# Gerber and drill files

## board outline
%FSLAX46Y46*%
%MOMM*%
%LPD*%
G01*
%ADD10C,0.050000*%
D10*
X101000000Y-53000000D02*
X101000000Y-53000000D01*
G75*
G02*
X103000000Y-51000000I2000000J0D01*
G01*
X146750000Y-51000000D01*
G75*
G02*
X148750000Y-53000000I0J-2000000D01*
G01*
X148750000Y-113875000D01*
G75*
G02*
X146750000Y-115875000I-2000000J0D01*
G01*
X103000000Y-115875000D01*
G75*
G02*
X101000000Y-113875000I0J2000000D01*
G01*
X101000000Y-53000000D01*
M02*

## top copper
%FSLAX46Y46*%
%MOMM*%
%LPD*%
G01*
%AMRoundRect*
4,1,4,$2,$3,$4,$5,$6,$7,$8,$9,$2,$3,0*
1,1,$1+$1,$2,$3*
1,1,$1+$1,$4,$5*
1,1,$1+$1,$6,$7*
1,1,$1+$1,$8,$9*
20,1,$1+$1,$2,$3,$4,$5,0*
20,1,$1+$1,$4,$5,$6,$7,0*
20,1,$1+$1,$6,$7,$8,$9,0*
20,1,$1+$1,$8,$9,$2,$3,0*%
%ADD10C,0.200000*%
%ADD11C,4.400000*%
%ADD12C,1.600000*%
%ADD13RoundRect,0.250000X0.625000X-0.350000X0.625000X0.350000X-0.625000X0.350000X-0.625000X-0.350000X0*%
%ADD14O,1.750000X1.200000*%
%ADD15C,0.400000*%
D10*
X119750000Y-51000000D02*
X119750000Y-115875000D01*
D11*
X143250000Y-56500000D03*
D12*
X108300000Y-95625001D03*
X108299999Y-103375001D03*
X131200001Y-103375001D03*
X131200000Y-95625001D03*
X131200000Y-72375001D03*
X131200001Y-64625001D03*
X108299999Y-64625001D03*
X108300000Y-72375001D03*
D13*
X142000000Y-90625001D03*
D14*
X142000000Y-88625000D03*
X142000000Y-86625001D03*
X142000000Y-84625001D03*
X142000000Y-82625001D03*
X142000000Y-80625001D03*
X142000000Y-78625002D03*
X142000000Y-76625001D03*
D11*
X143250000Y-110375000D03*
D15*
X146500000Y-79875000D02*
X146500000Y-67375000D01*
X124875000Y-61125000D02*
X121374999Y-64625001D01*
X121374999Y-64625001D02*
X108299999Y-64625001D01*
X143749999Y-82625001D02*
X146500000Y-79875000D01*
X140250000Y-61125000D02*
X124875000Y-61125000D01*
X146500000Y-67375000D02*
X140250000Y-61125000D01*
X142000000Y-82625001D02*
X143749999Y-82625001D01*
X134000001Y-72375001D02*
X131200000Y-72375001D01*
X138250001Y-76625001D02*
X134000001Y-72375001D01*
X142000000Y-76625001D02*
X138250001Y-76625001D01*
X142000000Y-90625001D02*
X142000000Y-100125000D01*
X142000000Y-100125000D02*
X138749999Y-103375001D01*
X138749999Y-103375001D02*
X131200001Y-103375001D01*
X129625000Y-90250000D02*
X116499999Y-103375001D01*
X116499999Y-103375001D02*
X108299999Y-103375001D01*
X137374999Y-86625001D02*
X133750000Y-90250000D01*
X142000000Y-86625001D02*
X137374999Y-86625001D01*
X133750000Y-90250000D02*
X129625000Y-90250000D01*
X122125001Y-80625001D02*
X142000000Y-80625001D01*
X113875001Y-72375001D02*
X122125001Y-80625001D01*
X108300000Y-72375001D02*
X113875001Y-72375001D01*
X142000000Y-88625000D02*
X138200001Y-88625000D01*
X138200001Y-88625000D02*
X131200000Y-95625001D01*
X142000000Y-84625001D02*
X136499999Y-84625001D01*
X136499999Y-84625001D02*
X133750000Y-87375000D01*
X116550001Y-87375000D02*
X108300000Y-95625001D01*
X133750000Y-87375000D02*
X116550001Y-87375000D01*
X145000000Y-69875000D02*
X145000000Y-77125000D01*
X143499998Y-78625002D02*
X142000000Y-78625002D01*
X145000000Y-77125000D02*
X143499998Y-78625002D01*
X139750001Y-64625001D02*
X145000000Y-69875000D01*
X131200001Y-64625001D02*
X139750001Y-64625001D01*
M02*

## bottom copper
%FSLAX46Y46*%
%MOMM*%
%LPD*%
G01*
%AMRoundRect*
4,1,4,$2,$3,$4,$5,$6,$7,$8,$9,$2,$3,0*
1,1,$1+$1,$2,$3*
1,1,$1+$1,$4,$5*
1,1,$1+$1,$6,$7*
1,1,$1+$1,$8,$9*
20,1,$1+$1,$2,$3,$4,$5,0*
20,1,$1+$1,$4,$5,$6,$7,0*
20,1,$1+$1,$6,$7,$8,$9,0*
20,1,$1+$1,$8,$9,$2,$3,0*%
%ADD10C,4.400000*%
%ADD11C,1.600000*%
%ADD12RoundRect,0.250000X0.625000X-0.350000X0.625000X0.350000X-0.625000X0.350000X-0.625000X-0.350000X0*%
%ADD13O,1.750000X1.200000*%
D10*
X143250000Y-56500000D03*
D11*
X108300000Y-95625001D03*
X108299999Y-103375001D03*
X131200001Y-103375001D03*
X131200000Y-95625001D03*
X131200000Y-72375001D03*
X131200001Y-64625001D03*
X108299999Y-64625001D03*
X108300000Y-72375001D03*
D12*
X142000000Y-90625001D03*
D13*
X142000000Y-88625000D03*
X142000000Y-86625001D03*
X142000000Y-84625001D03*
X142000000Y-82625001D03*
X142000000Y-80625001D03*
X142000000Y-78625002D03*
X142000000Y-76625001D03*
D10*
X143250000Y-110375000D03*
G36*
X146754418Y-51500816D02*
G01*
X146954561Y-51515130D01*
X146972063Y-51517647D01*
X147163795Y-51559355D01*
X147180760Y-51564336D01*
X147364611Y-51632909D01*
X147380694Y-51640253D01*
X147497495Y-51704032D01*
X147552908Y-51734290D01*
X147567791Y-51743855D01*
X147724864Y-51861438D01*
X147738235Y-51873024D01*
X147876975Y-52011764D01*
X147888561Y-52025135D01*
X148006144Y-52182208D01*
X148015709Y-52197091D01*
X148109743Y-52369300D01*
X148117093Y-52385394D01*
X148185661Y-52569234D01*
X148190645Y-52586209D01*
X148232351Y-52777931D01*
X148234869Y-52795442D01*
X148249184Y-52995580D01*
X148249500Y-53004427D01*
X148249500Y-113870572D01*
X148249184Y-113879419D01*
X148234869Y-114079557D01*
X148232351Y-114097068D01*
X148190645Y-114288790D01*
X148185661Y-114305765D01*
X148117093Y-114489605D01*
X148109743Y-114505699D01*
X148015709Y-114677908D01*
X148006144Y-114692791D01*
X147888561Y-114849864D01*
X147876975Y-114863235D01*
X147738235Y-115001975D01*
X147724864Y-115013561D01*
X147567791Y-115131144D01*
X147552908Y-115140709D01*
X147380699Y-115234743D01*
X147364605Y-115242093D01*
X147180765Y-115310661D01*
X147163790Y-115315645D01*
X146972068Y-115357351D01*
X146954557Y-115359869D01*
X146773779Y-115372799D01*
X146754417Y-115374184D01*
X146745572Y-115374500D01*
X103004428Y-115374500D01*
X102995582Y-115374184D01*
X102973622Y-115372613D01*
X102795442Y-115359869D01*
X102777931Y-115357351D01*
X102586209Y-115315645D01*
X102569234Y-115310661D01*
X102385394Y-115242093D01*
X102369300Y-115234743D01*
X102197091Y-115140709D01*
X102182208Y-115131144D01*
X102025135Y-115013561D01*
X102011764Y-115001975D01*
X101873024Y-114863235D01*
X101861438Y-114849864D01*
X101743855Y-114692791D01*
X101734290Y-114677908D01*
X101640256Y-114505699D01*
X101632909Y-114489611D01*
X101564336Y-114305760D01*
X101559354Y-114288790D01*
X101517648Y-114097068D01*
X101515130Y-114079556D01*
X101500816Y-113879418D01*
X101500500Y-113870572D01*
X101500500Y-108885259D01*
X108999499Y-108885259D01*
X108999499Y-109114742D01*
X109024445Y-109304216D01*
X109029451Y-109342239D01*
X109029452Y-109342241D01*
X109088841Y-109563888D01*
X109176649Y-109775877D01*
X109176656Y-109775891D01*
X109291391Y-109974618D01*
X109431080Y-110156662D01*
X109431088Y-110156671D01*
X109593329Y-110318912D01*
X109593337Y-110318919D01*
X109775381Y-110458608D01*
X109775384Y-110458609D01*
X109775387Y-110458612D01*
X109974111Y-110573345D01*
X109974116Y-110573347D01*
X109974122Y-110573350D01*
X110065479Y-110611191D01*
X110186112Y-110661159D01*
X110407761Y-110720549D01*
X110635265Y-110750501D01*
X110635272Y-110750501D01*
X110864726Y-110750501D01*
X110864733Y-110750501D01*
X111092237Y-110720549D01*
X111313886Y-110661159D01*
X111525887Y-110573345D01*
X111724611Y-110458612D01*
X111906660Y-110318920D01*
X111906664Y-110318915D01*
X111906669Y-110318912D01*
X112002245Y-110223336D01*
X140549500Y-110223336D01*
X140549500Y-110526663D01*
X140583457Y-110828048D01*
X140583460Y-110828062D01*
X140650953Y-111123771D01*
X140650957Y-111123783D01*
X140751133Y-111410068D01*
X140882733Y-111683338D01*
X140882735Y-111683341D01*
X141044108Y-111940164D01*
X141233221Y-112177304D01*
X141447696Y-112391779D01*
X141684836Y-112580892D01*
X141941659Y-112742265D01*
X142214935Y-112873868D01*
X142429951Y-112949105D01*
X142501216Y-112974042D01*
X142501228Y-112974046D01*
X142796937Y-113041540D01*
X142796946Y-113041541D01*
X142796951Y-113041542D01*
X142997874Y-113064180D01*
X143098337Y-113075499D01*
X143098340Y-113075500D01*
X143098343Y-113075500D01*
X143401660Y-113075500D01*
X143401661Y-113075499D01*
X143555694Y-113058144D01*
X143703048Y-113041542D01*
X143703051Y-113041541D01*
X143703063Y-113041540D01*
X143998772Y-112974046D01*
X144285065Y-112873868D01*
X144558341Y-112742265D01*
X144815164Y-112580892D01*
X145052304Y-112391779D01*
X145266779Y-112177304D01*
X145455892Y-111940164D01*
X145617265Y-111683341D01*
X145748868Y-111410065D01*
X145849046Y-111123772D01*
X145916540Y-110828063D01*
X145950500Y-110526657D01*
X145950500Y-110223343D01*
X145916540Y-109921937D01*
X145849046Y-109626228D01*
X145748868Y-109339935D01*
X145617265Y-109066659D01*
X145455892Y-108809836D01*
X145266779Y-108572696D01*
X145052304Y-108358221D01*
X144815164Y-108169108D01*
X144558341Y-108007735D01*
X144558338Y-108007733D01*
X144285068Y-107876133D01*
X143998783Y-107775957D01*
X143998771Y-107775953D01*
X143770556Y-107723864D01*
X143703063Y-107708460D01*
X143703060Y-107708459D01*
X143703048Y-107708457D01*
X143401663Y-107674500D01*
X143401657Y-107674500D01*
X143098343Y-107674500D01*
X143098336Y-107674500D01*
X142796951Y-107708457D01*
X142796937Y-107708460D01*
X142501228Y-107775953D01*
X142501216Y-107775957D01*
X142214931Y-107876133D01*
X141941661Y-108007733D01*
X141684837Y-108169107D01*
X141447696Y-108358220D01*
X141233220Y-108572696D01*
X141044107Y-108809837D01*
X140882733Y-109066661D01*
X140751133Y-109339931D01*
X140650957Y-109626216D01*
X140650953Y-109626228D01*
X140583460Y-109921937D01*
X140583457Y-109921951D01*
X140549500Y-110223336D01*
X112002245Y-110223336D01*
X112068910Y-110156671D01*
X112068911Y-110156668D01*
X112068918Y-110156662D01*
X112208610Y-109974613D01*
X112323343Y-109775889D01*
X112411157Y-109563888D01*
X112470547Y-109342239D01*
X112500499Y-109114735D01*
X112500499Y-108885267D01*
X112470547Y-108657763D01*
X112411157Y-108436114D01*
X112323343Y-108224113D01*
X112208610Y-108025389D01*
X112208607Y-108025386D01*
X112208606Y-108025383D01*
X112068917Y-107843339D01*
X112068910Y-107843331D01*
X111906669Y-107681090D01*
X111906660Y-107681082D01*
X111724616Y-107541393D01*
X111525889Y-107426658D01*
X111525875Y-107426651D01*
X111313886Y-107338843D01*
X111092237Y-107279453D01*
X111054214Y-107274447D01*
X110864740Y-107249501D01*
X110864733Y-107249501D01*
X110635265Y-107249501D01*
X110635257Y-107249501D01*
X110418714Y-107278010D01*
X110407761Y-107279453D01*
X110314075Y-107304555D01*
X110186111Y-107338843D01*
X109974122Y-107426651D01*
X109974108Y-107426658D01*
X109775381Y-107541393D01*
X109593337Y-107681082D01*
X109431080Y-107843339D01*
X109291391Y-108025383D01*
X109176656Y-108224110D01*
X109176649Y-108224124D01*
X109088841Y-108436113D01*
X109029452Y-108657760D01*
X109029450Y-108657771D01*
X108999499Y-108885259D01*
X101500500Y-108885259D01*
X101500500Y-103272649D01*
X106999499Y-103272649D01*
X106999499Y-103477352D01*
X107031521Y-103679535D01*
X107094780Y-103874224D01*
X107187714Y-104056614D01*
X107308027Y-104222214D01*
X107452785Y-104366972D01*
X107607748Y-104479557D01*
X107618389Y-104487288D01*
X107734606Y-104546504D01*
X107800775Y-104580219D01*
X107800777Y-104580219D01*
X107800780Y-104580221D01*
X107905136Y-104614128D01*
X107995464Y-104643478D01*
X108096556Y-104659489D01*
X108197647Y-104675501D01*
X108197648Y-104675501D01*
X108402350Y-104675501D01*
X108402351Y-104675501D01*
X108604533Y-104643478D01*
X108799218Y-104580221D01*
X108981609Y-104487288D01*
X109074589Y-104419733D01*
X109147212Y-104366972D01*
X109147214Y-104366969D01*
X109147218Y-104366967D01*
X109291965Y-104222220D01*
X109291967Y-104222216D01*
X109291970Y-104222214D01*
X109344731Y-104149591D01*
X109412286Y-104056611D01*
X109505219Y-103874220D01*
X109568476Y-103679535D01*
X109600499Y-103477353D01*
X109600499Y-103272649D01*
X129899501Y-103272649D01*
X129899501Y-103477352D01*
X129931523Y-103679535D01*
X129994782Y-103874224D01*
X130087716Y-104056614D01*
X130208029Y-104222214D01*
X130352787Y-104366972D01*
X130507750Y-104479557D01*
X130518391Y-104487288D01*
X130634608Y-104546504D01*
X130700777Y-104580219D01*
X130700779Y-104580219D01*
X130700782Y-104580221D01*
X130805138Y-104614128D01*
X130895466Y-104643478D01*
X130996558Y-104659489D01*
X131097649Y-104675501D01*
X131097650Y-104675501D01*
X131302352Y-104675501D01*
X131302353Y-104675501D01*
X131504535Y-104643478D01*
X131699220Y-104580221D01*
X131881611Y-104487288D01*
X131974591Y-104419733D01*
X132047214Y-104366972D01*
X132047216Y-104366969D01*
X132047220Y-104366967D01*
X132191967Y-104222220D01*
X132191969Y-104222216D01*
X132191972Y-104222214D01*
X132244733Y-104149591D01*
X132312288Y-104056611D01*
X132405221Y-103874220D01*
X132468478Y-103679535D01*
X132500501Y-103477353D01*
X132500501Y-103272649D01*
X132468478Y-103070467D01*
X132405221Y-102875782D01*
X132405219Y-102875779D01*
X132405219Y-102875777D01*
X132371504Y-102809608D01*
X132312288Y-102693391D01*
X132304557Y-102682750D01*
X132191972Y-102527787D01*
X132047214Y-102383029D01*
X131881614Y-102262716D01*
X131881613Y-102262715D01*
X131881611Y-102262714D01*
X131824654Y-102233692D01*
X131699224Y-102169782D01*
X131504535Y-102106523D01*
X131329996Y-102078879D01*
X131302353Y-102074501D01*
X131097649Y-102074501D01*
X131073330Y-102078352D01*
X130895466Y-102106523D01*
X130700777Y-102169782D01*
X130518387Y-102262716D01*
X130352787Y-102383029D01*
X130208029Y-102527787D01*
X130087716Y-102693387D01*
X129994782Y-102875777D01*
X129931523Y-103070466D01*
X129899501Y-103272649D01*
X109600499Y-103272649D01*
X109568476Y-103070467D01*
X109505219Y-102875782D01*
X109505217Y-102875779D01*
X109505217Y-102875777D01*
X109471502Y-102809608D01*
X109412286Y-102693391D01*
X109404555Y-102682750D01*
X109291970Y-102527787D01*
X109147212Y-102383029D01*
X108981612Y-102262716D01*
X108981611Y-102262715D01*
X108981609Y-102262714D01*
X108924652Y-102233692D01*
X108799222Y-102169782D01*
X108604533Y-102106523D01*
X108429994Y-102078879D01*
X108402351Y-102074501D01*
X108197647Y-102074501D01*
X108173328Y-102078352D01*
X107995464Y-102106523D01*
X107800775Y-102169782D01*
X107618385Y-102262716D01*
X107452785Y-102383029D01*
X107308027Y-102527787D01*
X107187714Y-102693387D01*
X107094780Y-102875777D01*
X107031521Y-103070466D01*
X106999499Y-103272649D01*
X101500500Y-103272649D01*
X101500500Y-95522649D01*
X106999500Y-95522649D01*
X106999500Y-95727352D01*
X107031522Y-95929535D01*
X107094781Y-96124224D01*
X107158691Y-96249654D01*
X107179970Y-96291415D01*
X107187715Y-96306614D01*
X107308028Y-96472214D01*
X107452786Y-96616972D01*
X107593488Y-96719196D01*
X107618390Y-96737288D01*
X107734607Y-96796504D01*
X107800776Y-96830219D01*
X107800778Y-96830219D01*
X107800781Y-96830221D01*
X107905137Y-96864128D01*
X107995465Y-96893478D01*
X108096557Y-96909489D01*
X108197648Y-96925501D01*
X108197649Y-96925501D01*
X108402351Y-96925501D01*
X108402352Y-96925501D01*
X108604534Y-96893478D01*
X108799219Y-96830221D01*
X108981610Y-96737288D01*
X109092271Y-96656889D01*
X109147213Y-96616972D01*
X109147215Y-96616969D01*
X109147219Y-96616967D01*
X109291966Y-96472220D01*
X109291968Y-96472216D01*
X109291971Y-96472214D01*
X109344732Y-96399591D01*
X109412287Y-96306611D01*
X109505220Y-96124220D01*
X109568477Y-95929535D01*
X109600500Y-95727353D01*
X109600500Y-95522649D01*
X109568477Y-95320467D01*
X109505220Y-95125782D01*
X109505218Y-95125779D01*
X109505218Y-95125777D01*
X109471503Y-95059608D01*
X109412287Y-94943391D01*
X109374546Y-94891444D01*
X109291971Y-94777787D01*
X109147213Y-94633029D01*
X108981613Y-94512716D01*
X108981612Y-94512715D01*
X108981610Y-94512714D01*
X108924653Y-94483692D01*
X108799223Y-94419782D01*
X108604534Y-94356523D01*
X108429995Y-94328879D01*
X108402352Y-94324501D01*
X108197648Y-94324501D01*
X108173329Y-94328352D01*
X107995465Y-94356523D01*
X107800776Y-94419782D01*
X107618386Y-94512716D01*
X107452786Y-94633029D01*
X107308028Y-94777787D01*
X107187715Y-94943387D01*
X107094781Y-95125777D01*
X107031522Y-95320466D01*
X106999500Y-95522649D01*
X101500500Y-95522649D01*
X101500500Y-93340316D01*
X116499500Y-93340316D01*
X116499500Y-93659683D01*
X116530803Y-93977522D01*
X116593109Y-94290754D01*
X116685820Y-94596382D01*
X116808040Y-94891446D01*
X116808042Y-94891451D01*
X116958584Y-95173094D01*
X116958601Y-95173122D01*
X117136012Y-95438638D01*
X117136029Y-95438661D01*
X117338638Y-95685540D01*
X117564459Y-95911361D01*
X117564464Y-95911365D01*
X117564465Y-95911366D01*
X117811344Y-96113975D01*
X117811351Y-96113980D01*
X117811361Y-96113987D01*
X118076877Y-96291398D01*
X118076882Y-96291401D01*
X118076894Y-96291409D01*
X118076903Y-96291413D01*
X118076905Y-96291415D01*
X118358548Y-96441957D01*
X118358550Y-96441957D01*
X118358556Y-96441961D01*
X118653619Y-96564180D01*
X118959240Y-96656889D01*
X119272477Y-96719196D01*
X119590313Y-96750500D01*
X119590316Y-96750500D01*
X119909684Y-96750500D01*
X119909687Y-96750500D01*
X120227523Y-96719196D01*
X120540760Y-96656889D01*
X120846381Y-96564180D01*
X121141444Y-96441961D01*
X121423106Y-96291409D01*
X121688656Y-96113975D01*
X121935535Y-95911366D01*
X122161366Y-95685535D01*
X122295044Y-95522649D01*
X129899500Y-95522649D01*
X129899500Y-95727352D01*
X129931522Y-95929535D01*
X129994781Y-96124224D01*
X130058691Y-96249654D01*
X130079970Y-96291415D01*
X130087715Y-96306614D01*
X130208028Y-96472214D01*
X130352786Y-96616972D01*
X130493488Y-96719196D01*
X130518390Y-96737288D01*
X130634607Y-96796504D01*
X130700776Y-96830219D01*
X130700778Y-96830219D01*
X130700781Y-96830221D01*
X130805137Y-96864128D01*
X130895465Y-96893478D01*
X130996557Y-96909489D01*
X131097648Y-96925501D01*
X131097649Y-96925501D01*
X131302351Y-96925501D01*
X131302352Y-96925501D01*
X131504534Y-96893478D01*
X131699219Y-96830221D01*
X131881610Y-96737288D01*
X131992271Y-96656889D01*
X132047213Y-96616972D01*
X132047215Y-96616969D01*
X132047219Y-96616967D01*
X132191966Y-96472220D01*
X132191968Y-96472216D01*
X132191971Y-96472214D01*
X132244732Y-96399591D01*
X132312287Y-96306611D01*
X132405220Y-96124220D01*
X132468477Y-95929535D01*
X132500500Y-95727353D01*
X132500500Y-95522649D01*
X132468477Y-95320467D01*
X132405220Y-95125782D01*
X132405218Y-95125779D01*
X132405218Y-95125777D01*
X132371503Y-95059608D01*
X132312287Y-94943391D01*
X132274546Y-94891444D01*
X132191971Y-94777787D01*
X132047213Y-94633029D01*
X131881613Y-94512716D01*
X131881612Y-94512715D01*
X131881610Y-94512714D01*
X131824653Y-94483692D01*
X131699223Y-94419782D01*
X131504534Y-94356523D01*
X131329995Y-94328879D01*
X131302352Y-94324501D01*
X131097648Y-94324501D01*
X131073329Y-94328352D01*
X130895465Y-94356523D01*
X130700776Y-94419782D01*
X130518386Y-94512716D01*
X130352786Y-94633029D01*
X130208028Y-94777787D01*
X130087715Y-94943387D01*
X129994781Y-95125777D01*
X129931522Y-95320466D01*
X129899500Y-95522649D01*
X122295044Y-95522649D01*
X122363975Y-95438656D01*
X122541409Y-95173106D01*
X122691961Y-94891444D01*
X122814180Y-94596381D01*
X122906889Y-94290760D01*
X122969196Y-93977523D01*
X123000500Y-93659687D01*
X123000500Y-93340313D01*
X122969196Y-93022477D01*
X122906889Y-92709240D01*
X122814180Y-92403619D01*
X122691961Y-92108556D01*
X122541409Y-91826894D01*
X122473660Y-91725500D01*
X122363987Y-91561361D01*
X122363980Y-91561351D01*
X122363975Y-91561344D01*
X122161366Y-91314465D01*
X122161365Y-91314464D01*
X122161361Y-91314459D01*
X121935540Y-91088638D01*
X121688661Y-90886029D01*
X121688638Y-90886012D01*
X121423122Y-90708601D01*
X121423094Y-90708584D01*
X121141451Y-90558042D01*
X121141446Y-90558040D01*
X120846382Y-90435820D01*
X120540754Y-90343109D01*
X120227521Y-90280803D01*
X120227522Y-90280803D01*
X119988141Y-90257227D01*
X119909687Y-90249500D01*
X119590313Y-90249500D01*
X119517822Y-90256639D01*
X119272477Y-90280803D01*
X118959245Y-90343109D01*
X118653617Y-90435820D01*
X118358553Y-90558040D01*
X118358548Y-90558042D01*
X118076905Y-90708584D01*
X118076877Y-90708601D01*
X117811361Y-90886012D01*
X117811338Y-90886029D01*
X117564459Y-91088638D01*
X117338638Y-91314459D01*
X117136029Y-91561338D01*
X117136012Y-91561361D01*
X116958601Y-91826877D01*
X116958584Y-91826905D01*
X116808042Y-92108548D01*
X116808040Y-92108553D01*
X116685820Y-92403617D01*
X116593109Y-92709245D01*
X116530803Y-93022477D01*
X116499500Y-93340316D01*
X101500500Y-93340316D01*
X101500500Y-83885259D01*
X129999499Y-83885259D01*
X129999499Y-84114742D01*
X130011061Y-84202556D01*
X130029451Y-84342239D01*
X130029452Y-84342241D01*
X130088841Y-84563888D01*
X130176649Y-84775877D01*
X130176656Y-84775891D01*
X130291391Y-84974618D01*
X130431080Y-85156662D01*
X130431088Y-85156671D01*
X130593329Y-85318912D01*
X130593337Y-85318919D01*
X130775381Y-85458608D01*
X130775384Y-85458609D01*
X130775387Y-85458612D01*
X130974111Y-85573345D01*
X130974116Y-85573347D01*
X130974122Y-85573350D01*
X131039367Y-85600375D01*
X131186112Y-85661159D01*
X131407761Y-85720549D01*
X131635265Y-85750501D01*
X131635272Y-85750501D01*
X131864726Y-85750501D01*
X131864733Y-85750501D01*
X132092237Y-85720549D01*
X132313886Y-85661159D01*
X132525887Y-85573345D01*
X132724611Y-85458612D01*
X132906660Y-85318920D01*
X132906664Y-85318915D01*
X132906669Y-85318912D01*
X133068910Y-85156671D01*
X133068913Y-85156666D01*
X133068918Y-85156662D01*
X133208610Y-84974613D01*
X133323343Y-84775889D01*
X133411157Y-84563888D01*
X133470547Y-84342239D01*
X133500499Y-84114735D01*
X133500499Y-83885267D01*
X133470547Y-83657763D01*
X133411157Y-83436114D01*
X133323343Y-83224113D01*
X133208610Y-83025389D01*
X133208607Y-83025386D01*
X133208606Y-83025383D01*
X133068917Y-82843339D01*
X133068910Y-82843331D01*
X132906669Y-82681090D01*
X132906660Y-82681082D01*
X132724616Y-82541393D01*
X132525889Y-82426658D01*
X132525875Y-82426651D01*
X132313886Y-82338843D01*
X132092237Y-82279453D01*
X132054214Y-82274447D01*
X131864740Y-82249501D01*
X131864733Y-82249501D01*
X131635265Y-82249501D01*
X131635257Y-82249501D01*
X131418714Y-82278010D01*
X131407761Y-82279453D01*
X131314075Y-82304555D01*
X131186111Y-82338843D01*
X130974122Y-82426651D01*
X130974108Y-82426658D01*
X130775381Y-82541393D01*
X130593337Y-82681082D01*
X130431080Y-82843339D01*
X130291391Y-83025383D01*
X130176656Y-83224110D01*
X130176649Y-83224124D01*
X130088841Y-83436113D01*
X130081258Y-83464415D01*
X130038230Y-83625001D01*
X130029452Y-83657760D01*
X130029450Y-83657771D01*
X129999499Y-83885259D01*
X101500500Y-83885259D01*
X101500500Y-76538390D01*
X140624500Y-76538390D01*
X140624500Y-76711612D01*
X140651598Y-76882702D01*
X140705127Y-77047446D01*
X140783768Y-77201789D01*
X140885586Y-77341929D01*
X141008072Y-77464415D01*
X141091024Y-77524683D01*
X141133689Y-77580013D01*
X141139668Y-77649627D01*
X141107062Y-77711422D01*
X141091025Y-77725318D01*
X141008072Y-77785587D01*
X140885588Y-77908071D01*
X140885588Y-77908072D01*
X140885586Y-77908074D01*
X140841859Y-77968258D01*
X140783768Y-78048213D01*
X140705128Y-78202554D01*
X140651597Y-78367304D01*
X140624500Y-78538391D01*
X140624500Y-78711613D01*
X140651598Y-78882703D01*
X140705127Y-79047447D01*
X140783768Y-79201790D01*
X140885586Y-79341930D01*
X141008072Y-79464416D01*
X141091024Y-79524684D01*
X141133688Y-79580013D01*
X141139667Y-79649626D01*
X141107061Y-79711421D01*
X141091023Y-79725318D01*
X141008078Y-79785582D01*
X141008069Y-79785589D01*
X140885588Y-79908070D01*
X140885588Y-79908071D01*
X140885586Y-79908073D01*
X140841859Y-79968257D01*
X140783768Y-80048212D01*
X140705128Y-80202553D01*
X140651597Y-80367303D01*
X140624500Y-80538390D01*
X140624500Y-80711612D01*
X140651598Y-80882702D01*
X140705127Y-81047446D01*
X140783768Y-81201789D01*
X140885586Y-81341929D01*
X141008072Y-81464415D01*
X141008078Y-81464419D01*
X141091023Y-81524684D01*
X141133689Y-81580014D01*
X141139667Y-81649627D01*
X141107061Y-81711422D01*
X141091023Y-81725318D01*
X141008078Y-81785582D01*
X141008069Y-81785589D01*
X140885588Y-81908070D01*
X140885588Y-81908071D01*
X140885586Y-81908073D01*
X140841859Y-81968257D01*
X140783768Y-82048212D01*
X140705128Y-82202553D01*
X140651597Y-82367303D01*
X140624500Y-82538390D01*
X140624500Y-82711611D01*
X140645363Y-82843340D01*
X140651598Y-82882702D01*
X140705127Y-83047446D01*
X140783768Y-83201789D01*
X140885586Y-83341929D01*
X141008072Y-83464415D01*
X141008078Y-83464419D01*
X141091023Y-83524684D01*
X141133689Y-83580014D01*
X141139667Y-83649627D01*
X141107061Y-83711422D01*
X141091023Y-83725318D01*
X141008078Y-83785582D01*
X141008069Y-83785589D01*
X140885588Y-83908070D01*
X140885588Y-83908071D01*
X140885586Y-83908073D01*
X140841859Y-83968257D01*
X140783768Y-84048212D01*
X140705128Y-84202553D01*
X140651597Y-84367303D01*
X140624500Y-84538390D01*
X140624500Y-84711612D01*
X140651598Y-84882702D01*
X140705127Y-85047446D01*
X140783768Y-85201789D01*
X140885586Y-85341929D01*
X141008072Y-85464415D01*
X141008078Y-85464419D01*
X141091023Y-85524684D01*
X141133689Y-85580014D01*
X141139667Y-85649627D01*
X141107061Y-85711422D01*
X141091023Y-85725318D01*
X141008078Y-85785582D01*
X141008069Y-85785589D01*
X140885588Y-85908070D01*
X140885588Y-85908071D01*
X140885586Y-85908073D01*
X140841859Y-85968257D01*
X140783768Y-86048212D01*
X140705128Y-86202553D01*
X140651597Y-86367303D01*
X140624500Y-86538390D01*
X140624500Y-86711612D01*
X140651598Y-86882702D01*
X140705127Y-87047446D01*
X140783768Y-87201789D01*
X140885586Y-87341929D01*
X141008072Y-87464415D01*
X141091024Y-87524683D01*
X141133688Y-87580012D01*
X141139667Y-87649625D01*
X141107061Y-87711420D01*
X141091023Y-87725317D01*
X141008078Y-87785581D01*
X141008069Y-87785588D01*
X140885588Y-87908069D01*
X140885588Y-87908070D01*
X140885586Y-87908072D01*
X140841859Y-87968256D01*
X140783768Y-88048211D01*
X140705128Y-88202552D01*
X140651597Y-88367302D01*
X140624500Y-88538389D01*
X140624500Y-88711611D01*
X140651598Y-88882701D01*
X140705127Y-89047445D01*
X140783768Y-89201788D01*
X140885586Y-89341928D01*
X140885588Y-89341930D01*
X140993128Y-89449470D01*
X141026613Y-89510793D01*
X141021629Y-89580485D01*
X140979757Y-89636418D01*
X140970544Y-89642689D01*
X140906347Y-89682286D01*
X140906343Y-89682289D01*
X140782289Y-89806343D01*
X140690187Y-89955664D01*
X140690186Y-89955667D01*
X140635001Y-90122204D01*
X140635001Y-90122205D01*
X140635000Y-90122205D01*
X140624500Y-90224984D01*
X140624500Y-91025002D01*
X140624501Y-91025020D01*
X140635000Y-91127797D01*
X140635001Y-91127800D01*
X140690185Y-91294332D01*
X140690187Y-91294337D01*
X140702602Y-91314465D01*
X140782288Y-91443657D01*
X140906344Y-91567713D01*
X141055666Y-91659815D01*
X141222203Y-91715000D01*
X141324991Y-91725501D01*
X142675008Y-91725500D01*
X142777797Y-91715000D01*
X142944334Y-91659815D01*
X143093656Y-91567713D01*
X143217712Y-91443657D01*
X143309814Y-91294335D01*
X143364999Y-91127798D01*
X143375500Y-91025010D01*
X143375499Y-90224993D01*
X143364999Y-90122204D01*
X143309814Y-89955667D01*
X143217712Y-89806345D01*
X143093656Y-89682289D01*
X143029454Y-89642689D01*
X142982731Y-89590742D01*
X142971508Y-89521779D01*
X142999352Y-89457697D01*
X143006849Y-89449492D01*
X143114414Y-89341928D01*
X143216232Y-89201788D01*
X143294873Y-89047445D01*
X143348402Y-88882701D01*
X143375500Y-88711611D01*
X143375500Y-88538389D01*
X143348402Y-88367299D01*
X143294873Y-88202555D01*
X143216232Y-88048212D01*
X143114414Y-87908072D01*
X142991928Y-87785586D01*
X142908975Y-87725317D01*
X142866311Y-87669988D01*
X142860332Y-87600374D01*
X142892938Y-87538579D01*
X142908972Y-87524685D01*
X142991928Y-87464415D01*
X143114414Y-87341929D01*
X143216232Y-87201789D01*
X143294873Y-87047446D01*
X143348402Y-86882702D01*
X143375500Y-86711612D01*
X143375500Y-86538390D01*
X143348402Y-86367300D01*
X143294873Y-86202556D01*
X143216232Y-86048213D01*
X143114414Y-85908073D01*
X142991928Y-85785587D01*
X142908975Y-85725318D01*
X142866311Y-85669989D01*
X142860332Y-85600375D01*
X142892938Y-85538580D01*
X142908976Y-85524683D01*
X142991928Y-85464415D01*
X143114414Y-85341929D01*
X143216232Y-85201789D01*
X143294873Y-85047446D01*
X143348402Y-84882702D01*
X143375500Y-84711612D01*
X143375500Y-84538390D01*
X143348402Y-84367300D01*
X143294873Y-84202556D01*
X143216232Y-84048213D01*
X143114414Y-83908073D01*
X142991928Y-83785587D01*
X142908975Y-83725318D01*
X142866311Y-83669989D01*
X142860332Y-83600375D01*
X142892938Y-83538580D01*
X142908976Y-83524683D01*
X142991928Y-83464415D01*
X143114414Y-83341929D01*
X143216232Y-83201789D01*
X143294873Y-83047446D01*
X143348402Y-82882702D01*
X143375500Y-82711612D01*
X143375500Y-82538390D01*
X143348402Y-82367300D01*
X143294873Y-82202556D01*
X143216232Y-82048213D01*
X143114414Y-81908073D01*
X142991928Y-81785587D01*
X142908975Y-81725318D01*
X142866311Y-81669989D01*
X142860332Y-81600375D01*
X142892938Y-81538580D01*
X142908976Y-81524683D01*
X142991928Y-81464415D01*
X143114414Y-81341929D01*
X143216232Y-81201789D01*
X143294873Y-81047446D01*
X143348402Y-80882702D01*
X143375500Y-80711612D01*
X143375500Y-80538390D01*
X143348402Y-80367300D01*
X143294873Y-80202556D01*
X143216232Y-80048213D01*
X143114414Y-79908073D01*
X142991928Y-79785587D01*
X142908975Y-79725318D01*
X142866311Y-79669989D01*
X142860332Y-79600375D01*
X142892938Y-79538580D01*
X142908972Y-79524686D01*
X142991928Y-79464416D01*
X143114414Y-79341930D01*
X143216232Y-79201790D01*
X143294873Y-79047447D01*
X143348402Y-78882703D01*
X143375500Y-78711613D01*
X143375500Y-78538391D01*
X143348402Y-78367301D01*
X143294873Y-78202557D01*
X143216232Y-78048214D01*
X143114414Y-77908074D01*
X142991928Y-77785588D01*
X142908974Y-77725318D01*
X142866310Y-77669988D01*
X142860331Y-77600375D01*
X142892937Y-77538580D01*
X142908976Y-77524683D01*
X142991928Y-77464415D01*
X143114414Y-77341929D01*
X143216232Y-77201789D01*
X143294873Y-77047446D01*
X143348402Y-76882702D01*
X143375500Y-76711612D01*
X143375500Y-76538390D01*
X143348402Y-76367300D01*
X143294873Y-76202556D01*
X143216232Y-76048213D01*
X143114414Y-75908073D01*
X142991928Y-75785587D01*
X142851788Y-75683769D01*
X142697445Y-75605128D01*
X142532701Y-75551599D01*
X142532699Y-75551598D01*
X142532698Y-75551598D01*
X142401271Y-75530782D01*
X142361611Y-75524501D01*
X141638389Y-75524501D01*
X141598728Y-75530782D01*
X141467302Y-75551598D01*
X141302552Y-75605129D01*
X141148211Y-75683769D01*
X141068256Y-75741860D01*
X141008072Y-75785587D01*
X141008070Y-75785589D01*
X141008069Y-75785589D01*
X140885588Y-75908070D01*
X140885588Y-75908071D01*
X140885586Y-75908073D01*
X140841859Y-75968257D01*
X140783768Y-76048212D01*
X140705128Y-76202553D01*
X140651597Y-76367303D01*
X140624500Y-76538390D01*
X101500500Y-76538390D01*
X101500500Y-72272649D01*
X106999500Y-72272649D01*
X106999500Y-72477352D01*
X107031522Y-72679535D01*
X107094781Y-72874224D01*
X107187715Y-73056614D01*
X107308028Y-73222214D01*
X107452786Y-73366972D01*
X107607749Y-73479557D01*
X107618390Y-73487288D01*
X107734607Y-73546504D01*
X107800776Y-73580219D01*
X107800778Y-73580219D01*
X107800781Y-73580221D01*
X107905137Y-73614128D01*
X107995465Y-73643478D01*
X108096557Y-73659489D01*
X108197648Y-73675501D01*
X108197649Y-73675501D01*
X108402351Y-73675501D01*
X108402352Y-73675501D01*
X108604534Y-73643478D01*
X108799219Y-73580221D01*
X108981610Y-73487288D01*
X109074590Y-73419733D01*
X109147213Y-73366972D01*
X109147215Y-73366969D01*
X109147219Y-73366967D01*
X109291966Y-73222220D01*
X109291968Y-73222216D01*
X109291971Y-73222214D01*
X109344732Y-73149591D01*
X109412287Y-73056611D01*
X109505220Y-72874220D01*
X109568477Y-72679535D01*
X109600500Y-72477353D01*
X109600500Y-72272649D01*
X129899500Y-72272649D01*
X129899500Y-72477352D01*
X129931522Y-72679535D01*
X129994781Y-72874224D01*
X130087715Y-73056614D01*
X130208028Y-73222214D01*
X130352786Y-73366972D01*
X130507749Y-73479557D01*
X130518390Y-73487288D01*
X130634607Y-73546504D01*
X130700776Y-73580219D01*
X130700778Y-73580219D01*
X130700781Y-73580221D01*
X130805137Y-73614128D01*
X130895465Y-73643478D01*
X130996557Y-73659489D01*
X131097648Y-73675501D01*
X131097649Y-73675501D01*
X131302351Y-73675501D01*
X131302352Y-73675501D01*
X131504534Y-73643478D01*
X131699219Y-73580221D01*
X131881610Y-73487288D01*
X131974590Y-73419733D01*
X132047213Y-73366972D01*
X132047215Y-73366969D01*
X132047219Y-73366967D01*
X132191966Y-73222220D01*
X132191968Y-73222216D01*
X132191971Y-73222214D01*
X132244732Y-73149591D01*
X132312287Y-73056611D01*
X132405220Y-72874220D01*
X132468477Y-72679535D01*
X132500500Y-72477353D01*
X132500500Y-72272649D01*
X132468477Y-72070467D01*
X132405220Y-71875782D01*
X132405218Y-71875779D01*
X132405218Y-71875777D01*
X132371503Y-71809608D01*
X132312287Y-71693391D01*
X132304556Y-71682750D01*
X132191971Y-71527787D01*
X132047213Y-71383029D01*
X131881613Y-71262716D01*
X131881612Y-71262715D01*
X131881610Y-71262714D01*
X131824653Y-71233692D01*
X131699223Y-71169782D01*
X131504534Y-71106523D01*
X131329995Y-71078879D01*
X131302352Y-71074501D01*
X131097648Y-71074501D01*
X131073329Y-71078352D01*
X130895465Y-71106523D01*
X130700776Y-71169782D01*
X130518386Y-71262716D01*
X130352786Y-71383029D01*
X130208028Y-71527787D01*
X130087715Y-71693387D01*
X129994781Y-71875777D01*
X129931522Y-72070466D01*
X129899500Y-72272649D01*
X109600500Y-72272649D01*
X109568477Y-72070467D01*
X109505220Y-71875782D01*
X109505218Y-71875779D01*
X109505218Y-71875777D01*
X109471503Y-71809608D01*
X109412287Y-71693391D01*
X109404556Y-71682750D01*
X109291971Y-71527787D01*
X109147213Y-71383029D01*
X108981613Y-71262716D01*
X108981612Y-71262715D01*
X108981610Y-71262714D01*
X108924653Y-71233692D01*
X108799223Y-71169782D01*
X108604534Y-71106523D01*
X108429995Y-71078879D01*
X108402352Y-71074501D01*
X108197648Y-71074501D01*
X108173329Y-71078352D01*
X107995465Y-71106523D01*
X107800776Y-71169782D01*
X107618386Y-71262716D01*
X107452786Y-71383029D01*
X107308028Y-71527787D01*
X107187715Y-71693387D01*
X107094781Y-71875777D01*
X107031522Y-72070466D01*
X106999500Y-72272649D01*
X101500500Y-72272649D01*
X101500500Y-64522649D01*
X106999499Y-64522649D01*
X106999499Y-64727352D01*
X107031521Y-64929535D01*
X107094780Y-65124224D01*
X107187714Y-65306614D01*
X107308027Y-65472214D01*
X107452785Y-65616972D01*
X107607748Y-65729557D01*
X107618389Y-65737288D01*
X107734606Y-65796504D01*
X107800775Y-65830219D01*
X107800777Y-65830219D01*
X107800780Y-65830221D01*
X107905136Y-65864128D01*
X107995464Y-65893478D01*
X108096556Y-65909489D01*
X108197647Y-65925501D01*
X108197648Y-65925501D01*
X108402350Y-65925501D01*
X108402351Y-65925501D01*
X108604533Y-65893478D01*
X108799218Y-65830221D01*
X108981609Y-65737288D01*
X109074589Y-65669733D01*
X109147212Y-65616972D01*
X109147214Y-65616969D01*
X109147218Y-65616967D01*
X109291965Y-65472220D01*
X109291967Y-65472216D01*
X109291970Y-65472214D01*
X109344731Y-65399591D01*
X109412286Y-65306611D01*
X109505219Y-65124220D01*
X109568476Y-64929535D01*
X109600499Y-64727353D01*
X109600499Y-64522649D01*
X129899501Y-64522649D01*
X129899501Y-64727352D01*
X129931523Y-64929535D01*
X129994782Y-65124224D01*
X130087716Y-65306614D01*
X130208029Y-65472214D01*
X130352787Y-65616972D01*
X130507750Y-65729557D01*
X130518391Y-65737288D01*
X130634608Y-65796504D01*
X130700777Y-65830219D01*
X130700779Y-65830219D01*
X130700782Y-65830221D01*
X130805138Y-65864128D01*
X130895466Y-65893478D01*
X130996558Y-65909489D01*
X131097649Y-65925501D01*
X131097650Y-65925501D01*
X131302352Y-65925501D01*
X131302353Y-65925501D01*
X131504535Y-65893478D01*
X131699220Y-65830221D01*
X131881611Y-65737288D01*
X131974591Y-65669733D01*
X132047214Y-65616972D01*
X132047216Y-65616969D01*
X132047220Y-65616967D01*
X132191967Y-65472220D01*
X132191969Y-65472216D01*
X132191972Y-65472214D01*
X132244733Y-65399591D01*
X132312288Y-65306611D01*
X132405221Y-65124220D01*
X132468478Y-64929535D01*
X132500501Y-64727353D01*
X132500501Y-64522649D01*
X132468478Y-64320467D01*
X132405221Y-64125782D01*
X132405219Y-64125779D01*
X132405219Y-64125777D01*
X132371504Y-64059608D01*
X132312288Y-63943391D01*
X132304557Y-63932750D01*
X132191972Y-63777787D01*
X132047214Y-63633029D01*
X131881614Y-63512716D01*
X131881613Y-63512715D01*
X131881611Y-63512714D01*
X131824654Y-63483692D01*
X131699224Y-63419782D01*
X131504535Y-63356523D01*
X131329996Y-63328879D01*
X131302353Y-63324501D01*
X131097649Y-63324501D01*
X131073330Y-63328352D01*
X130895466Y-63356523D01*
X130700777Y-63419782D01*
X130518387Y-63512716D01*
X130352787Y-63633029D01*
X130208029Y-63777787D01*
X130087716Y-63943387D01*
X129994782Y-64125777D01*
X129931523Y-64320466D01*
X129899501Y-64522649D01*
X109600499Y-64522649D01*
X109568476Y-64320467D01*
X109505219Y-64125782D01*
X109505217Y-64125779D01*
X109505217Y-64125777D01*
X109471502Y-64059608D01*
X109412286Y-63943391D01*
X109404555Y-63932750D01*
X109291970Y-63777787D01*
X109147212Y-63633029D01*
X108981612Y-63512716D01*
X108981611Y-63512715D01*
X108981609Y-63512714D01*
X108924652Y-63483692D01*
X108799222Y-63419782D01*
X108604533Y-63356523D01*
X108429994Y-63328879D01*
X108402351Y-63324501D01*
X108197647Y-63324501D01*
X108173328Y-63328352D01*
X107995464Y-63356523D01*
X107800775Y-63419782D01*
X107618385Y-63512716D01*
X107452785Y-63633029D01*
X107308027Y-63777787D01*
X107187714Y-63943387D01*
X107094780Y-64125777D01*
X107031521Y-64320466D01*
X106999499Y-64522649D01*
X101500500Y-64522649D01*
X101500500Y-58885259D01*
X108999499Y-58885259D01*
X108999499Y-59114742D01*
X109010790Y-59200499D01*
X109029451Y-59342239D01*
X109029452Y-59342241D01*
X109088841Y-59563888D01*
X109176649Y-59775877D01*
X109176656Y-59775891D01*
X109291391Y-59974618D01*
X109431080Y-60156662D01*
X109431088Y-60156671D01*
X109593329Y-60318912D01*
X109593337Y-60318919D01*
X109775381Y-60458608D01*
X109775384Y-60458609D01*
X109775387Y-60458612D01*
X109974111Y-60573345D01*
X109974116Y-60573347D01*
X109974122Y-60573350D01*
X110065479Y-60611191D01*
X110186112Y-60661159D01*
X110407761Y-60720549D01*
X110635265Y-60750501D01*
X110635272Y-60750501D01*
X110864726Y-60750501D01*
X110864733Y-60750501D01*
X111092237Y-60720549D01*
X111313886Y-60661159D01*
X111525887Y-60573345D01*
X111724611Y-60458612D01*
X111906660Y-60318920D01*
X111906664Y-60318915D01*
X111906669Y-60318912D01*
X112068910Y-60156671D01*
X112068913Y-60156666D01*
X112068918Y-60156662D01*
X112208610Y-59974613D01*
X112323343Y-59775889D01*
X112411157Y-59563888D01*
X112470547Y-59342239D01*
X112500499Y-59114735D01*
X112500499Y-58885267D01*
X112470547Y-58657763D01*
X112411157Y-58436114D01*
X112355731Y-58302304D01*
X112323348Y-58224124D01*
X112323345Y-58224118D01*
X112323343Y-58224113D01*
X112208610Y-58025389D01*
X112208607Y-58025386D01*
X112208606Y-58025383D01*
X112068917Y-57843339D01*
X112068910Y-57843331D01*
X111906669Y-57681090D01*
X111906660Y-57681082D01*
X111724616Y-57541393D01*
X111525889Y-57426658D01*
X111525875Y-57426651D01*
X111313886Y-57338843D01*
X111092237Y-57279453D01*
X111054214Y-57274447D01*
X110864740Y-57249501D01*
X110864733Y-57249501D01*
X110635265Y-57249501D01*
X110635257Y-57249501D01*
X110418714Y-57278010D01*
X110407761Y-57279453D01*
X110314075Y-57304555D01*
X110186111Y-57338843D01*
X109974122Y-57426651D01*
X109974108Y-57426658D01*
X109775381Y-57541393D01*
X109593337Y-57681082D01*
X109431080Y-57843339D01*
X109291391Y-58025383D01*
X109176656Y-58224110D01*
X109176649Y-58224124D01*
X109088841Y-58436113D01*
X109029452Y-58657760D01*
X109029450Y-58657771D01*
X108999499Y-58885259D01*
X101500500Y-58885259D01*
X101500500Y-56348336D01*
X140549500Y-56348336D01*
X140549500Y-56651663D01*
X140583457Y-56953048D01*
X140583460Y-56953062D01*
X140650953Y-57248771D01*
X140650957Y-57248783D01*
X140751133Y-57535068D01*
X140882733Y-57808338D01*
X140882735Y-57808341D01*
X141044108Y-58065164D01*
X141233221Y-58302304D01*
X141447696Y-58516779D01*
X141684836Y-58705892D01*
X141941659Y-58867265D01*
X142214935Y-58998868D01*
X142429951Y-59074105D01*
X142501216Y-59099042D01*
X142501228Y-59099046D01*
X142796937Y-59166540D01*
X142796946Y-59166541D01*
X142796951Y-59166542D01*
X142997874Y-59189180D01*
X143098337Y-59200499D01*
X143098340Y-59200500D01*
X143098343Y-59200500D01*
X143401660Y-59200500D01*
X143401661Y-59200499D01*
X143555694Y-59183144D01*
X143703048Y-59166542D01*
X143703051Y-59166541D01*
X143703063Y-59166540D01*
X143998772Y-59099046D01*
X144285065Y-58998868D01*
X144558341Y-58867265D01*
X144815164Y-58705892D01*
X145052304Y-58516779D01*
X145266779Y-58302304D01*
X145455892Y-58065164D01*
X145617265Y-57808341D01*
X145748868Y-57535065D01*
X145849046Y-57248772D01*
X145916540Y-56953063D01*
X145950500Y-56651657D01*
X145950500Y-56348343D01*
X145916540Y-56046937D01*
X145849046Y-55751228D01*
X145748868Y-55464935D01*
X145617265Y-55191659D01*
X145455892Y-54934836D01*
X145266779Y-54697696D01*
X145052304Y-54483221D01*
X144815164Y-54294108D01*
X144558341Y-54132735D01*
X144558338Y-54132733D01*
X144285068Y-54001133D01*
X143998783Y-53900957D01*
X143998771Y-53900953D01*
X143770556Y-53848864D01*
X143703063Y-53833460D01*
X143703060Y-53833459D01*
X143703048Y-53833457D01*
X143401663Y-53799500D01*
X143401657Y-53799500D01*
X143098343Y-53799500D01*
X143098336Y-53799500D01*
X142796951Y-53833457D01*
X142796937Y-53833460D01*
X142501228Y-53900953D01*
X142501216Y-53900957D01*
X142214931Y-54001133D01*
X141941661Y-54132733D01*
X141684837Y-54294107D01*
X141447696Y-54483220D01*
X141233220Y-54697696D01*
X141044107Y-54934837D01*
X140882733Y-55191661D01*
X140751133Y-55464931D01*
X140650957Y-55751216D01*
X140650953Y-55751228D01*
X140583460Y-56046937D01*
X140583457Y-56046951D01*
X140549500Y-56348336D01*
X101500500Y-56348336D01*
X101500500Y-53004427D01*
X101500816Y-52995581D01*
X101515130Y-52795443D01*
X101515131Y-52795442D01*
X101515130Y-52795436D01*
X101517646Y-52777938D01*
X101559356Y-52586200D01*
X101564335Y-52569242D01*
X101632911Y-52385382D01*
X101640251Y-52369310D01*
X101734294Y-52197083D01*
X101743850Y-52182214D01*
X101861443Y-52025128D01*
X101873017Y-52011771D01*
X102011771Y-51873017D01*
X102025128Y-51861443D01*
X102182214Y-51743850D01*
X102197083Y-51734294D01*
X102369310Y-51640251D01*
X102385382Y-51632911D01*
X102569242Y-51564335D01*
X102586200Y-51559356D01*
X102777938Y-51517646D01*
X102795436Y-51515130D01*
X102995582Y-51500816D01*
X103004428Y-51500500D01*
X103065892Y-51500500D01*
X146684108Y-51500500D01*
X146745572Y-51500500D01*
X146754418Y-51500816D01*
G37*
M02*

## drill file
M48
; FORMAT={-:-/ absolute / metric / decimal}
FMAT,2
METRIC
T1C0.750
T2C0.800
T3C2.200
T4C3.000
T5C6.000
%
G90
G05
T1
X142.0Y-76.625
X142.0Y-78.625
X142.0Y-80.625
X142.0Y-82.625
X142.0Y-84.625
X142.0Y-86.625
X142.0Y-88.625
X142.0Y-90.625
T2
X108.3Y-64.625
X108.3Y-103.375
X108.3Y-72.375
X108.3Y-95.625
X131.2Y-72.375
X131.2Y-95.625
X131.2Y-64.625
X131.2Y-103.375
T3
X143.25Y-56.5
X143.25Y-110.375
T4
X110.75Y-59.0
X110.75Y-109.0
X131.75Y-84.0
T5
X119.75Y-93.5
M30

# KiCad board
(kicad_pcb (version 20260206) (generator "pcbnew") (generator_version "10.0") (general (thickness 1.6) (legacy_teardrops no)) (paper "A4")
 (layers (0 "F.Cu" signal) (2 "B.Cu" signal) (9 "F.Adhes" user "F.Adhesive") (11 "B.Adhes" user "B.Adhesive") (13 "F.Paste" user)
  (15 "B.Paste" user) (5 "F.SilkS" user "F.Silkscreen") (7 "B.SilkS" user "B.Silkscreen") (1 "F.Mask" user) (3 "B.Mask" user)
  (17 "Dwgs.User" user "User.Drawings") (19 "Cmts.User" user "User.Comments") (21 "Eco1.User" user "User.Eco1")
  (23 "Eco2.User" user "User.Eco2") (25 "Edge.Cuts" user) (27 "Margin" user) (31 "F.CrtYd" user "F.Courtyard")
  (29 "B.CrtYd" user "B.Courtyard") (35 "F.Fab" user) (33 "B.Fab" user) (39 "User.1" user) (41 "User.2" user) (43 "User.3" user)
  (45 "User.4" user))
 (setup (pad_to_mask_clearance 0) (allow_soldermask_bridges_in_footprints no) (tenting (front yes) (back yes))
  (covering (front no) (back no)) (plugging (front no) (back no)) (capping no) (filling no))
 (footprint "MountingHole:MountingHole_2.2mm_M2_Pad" (layer "F.Cu") (at 143.25 56.5)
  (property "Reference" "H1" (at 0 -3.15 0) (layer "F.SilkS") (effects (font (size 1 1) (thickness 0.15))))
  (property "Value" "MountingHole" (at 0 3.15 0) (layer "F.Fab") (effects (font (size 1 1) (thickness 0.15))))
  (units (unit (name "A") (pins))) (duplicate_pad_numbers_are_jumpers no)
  (pad "1" thru_hole circle (at 0 0) (size 4.4 4.4) (drill 2.2) (layers "*.Cu" "*.Mask") (remove_unused_layers no) (zone_connect 2)))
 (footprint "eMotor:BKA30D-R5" (layer "F.Cu") (at 119.75 84.000001 90)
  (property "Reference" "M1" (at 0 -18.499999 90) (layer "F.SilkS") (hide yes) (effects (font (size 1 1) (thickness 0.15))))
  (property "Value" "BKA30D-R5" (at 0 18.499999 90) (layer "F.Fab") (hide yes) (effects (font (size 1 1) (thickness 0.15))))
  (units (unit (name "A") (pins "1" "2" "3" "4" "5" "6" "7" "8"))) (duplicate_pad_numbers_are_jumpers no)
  (pad "" np_thru_hole circle (at -25 -9.000001 90) (size 3 3) (drill 3) (layers "*.Cu" "*.Mask"))
  (pad "" np_thru_hole circle (at -9.499999 0 90) (size 6 6) (drill 6) (layers "*.Cu" "*.Mask"))
  (pad "" np_thru_hole circle (at 0 11.999999 90) (size 3 3) (drill 3) (layers "*.Cu" "*.Mask"))
  (pad "" np_thru_hole circle (at 25 -9.000001 90) (size 3 3) (drill 3) (layers "*.Cu" "*.Mask"))
  (pad "1" thru_hole circle (at -11.625 -11.45 90) (size 1.6 1.6) (drill 0.8) (layers "*.Cu" "*.Mask") (remove_unused_layers no)
   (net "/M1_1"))
  (pad "2" thru_hole circle (at -19.375 -11.450001 90) (size 1.6 1.6) (drill 0.8) (layers "*.Cu" "*.Mask") (remove_unused_layers no)
   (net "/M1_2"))
  (pad "3" thru_hole circle (at -19.375 11.450001 90) (size 1.6 1.6) (drill 0.8) (layers "*.Cu" "*.Mask") (remove_unused_layers no)
   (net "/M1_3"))
  (pad "4" thru_hole circle (at -11.625 11.45 90) (size 1.6 1.6) (drill 0.8) (layers "*.Cu" "*.Mask") (remove_unused_layers no)
   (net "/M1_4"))
  (pad "5" thru_hole circle (at 11.625 11.45 90) (size 1.6 1.6) (drill 0.8) (layers "*.Cu" "*.Mask") (remove_unused_layers no) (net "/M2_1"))
  (pad "6" thru_hole circle (at 19.375 11.450001 90) (size 1.6 1.6) (drill 0.8) (layers "*.Cu" "*.Mask") (remove_unused_layers no)
   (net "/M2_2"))
  (pad "7" thru_hole circle (at 19.375 -11.450001 90) (size 1.6 1.6) (drill 0.8) (layers "*.Cu" "*.Mask") (remove_unused_layers no)
   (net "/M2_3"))
  (pad "8" thru_hole circle (at 11.625 -11.45 90) (size 1.6 1.6) (drill 0.8) (layers "*.Cu" "*.Mask") (remove_unused_layers no)
   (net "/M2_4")))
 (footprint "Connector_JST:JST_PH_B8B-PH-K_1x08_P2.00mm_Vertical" (layer "F.Cu") (at 142 90.625001 90)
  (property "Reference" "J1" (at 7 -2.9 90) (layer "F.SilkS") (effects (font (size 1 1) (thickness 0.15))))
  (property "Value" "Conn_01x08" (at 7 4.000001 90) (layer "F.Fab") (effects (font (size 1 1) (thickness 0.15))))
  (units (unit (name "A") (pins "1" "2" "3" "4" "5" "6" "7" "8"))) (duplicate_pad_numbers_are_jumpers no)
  (pad "1" thru_hole roundrect (at 0 0 90) (size 1.2 1.75) (drill 0.75) (layers "*.Cu" "*.Mask") (remove_unused_layers no)
   (roundrect_rratio 0.208333) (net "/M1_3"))
  (pad "2" thru_hole oval (at 2.000001 0 90) (size 1.2 1.75) (drill 0.75) (layers "*.Cu" "*.Mask") (remove_unused_layers no) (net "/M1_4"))
  (pad "3" thru_hole oval (at 4 0 90) (size 1.2 1.75) (drill 0.75) (layers "*.Cu" "*.Mask") (remove_unused_layers no) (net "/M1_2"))
  (pad "4" thru_hole oval (at 6 0 90) (size 1.2 1.75) (drill 0.75) (layers "*.Cu" "*.Mask") (remove_unused_layers no) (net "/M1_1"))
  (pad "5" thru_hole oval (at 8 0 90) (size 1.2 1.75) (drill 0.75) (layers "*.Cu" "*.Mask") (remove_unused_layers no) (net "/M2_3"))
  (pad "6" thru_hole oval (at 10 0 90) (size 1.2 1.75) (drill 0.75) (layers "*.Cu" "*.Mask") (remove_unused_layers no) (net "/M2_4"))
  (pad "7" thru_hole oval (at 11.999999 0 90) (size 1.2 1.75) (drill 0.75) (layers "*.Cu" "*.Mask") (remove_unused_layers no) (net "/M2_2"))
  (pad "8" thru_hole oval (at 14 0 90) (size 1.2 1.75) (drill 0.75) (layers "*.Cu" "*.Mask") (remove_unused_layers no) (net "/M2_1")))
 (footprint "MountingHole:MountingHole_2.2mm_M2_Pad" (layer "F.Cu") (at 143.25 110.375)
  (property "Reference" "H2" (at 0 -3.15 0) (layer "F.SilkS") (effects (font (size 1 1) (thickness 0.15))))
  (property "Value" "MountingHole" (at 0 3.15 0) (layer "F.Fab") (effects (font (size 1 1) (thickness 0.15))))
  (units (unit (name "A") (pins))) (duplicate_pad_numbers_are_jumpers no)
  (pad "1" thru_hole circle (at 0 0) (size 4.4 4.4) (drill 2.2) (layers "*.Cu" "*.Mask") (remove_unused_layers no) (zone_connect 2)))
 (gr_line (start 119.75 51) (end 119.75 115.875) (stroke (width 0.2) (type default)) (layer "F.Cu"))
 (gr_rect (start 101 51) (end 148.75 115.875) (radius 2) (stroke (width 0.05) (type solid)) (fill no) (layer "Edge.Cuts"))
 (segment (start 146.5 79.875) (end 146.5 67.375) (width 0.4) (layer "F.Cu") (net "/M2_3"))
 (segment (start 124.875 61.125) (end 121.374999 64.625001) (width 0.4) (layer "F.Cu") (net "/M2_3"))
 (segment (start 121.374999 64.625001) (end 108.299999 64.625001) (width 0.4) (layer "F.Cu") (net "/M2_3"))
 (segment (start 143.749999 82.625001) (end 146.5 79.875) (width 0.4) (layer "F.Cu") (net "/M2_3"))
 (segment (start 140.25 61.125) (end 124.875 61.125) (width 0.4) (layer "F.Cu") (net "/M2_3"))
 (segment (start 146.5 67.375) (end 140.25 61.125) (width 0.4) (layer "F.Cu") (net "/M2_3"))
 (segment (start 142 82.625001) (end 143.749999 82.625001) (width 0.4) (layer "F.Cu") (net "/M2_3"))
 (segment (start 134.000001 72.375001) (end 131.2 72.375001) (width 0.4) (layer "F.Cu") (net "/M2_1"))
 (segment (start 138.250001 76.625001) (end 134.000001 72.375001) (width 0.4) (layer "F.Cu") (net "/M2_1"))
 (segment (start 142 76.625001) (end 138.250001 76.625001) (width 0.4) (layer "F.Cu") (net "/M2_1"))
 (segment (start 142 90.625001) (end 142 100.125) (width 0.4) (layer "F.Cu") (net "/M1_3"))
 (segment (start 142 100.125) (end 138.749999 103.375001) (width 0.4) (layer "F.Cu") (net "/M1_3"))
 (segment (start 138.749999 103.375001) (end 131.200001 103.375001) (width 0.4) (layer "F.Cu") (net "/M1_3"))
 (segment (start 129.625 90.25) (end 116.499999 103.375001) (width 0.4) (layer "F.Cu") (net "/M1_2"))
 (segment (start 116.499999 103.375001) (end 108.299999 103.375001) (width 0.4) (layer "F.Cu") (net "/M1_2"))
 (segment (start 137.374999 86.625001) (end 133.75 90.25) (width 0.4) (layer "F.Cu") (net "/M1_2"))
 (segment (start 142 86.625001) (end 137.374999 86.625001) (width 0.4) (layer "F.Cu") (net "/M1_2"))
 (segment (start 133.75 90.25) (end 129.625 90.25) (width 0.4) (layer "F.Cu") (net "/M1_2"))
 (segment (start 122.125001 80.625001) (end 142 80.625001) (width 0.4) (layer "F.Cu") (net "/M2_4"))
 (segment (start 113.875001 72.375001) (end 122.125001 80.625001) (width 0.4) (layer "F.Cu") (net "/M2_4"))
 (segment (start 108.3 72.375001) (end 113.875001 72.375001) (width 0.4) (layer "F.Cu") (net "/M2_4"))
 (segment (start 142 88.625) (end 138.200001 88.625) (width 0.4) (layer "F.Cu") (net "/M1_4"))
 (segment (start 138.200001 88.625) (end 131.2 95.625001) (width 0.4) (layer "F.Cu") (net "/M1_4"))
 (segment (start 142 84.625001) (end 136.499999 84.625001) (width 0.4) (layer "F.Cu") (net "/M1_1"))
 (segment (start 136.499999 84.625001) (end 133.75 87.375) (width 0.4) (layer "F.Cu") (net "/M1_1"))
 (segment (start 116.550001 87.375) (end 108.3 95.625001) (width 0.4) (layer "F.Cu") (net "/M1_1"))
 (segment (start 133.75 87.375) (end 116.550001 87.375) (width 0.4) (layer "F.Cu") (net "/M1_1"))
 (segment (start 145 69.875) (end 145 77.125) (width 0.4) (layer "F.Cu") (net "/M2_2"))
 (segment (start 143.499998 78.625002) (end 142 78.625002) (width 0.4) (layer "F.Cu") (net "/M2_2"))
 (segment (start 145 77.125) (end 143.499998 78.625002) (width 0.4) (layer "F.Cu") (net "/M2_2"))
 (segment (start 139.750001 64.625001) (end 145 69.875) (width 0.4) (layer "F.Cu") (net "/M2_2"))
 (segment (start 131.200001 64.625001) (end 139.750001 64.625001) (width 0.4) (layer "F.Cu") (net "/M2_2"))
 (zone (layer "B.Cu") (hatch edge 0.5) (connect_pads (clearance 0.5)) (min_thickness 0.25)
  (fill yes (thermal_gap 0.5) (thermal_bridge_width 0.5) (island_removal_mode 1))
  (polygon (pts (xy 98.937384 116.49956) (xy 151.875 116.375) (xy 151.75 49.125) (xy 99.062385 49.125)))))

